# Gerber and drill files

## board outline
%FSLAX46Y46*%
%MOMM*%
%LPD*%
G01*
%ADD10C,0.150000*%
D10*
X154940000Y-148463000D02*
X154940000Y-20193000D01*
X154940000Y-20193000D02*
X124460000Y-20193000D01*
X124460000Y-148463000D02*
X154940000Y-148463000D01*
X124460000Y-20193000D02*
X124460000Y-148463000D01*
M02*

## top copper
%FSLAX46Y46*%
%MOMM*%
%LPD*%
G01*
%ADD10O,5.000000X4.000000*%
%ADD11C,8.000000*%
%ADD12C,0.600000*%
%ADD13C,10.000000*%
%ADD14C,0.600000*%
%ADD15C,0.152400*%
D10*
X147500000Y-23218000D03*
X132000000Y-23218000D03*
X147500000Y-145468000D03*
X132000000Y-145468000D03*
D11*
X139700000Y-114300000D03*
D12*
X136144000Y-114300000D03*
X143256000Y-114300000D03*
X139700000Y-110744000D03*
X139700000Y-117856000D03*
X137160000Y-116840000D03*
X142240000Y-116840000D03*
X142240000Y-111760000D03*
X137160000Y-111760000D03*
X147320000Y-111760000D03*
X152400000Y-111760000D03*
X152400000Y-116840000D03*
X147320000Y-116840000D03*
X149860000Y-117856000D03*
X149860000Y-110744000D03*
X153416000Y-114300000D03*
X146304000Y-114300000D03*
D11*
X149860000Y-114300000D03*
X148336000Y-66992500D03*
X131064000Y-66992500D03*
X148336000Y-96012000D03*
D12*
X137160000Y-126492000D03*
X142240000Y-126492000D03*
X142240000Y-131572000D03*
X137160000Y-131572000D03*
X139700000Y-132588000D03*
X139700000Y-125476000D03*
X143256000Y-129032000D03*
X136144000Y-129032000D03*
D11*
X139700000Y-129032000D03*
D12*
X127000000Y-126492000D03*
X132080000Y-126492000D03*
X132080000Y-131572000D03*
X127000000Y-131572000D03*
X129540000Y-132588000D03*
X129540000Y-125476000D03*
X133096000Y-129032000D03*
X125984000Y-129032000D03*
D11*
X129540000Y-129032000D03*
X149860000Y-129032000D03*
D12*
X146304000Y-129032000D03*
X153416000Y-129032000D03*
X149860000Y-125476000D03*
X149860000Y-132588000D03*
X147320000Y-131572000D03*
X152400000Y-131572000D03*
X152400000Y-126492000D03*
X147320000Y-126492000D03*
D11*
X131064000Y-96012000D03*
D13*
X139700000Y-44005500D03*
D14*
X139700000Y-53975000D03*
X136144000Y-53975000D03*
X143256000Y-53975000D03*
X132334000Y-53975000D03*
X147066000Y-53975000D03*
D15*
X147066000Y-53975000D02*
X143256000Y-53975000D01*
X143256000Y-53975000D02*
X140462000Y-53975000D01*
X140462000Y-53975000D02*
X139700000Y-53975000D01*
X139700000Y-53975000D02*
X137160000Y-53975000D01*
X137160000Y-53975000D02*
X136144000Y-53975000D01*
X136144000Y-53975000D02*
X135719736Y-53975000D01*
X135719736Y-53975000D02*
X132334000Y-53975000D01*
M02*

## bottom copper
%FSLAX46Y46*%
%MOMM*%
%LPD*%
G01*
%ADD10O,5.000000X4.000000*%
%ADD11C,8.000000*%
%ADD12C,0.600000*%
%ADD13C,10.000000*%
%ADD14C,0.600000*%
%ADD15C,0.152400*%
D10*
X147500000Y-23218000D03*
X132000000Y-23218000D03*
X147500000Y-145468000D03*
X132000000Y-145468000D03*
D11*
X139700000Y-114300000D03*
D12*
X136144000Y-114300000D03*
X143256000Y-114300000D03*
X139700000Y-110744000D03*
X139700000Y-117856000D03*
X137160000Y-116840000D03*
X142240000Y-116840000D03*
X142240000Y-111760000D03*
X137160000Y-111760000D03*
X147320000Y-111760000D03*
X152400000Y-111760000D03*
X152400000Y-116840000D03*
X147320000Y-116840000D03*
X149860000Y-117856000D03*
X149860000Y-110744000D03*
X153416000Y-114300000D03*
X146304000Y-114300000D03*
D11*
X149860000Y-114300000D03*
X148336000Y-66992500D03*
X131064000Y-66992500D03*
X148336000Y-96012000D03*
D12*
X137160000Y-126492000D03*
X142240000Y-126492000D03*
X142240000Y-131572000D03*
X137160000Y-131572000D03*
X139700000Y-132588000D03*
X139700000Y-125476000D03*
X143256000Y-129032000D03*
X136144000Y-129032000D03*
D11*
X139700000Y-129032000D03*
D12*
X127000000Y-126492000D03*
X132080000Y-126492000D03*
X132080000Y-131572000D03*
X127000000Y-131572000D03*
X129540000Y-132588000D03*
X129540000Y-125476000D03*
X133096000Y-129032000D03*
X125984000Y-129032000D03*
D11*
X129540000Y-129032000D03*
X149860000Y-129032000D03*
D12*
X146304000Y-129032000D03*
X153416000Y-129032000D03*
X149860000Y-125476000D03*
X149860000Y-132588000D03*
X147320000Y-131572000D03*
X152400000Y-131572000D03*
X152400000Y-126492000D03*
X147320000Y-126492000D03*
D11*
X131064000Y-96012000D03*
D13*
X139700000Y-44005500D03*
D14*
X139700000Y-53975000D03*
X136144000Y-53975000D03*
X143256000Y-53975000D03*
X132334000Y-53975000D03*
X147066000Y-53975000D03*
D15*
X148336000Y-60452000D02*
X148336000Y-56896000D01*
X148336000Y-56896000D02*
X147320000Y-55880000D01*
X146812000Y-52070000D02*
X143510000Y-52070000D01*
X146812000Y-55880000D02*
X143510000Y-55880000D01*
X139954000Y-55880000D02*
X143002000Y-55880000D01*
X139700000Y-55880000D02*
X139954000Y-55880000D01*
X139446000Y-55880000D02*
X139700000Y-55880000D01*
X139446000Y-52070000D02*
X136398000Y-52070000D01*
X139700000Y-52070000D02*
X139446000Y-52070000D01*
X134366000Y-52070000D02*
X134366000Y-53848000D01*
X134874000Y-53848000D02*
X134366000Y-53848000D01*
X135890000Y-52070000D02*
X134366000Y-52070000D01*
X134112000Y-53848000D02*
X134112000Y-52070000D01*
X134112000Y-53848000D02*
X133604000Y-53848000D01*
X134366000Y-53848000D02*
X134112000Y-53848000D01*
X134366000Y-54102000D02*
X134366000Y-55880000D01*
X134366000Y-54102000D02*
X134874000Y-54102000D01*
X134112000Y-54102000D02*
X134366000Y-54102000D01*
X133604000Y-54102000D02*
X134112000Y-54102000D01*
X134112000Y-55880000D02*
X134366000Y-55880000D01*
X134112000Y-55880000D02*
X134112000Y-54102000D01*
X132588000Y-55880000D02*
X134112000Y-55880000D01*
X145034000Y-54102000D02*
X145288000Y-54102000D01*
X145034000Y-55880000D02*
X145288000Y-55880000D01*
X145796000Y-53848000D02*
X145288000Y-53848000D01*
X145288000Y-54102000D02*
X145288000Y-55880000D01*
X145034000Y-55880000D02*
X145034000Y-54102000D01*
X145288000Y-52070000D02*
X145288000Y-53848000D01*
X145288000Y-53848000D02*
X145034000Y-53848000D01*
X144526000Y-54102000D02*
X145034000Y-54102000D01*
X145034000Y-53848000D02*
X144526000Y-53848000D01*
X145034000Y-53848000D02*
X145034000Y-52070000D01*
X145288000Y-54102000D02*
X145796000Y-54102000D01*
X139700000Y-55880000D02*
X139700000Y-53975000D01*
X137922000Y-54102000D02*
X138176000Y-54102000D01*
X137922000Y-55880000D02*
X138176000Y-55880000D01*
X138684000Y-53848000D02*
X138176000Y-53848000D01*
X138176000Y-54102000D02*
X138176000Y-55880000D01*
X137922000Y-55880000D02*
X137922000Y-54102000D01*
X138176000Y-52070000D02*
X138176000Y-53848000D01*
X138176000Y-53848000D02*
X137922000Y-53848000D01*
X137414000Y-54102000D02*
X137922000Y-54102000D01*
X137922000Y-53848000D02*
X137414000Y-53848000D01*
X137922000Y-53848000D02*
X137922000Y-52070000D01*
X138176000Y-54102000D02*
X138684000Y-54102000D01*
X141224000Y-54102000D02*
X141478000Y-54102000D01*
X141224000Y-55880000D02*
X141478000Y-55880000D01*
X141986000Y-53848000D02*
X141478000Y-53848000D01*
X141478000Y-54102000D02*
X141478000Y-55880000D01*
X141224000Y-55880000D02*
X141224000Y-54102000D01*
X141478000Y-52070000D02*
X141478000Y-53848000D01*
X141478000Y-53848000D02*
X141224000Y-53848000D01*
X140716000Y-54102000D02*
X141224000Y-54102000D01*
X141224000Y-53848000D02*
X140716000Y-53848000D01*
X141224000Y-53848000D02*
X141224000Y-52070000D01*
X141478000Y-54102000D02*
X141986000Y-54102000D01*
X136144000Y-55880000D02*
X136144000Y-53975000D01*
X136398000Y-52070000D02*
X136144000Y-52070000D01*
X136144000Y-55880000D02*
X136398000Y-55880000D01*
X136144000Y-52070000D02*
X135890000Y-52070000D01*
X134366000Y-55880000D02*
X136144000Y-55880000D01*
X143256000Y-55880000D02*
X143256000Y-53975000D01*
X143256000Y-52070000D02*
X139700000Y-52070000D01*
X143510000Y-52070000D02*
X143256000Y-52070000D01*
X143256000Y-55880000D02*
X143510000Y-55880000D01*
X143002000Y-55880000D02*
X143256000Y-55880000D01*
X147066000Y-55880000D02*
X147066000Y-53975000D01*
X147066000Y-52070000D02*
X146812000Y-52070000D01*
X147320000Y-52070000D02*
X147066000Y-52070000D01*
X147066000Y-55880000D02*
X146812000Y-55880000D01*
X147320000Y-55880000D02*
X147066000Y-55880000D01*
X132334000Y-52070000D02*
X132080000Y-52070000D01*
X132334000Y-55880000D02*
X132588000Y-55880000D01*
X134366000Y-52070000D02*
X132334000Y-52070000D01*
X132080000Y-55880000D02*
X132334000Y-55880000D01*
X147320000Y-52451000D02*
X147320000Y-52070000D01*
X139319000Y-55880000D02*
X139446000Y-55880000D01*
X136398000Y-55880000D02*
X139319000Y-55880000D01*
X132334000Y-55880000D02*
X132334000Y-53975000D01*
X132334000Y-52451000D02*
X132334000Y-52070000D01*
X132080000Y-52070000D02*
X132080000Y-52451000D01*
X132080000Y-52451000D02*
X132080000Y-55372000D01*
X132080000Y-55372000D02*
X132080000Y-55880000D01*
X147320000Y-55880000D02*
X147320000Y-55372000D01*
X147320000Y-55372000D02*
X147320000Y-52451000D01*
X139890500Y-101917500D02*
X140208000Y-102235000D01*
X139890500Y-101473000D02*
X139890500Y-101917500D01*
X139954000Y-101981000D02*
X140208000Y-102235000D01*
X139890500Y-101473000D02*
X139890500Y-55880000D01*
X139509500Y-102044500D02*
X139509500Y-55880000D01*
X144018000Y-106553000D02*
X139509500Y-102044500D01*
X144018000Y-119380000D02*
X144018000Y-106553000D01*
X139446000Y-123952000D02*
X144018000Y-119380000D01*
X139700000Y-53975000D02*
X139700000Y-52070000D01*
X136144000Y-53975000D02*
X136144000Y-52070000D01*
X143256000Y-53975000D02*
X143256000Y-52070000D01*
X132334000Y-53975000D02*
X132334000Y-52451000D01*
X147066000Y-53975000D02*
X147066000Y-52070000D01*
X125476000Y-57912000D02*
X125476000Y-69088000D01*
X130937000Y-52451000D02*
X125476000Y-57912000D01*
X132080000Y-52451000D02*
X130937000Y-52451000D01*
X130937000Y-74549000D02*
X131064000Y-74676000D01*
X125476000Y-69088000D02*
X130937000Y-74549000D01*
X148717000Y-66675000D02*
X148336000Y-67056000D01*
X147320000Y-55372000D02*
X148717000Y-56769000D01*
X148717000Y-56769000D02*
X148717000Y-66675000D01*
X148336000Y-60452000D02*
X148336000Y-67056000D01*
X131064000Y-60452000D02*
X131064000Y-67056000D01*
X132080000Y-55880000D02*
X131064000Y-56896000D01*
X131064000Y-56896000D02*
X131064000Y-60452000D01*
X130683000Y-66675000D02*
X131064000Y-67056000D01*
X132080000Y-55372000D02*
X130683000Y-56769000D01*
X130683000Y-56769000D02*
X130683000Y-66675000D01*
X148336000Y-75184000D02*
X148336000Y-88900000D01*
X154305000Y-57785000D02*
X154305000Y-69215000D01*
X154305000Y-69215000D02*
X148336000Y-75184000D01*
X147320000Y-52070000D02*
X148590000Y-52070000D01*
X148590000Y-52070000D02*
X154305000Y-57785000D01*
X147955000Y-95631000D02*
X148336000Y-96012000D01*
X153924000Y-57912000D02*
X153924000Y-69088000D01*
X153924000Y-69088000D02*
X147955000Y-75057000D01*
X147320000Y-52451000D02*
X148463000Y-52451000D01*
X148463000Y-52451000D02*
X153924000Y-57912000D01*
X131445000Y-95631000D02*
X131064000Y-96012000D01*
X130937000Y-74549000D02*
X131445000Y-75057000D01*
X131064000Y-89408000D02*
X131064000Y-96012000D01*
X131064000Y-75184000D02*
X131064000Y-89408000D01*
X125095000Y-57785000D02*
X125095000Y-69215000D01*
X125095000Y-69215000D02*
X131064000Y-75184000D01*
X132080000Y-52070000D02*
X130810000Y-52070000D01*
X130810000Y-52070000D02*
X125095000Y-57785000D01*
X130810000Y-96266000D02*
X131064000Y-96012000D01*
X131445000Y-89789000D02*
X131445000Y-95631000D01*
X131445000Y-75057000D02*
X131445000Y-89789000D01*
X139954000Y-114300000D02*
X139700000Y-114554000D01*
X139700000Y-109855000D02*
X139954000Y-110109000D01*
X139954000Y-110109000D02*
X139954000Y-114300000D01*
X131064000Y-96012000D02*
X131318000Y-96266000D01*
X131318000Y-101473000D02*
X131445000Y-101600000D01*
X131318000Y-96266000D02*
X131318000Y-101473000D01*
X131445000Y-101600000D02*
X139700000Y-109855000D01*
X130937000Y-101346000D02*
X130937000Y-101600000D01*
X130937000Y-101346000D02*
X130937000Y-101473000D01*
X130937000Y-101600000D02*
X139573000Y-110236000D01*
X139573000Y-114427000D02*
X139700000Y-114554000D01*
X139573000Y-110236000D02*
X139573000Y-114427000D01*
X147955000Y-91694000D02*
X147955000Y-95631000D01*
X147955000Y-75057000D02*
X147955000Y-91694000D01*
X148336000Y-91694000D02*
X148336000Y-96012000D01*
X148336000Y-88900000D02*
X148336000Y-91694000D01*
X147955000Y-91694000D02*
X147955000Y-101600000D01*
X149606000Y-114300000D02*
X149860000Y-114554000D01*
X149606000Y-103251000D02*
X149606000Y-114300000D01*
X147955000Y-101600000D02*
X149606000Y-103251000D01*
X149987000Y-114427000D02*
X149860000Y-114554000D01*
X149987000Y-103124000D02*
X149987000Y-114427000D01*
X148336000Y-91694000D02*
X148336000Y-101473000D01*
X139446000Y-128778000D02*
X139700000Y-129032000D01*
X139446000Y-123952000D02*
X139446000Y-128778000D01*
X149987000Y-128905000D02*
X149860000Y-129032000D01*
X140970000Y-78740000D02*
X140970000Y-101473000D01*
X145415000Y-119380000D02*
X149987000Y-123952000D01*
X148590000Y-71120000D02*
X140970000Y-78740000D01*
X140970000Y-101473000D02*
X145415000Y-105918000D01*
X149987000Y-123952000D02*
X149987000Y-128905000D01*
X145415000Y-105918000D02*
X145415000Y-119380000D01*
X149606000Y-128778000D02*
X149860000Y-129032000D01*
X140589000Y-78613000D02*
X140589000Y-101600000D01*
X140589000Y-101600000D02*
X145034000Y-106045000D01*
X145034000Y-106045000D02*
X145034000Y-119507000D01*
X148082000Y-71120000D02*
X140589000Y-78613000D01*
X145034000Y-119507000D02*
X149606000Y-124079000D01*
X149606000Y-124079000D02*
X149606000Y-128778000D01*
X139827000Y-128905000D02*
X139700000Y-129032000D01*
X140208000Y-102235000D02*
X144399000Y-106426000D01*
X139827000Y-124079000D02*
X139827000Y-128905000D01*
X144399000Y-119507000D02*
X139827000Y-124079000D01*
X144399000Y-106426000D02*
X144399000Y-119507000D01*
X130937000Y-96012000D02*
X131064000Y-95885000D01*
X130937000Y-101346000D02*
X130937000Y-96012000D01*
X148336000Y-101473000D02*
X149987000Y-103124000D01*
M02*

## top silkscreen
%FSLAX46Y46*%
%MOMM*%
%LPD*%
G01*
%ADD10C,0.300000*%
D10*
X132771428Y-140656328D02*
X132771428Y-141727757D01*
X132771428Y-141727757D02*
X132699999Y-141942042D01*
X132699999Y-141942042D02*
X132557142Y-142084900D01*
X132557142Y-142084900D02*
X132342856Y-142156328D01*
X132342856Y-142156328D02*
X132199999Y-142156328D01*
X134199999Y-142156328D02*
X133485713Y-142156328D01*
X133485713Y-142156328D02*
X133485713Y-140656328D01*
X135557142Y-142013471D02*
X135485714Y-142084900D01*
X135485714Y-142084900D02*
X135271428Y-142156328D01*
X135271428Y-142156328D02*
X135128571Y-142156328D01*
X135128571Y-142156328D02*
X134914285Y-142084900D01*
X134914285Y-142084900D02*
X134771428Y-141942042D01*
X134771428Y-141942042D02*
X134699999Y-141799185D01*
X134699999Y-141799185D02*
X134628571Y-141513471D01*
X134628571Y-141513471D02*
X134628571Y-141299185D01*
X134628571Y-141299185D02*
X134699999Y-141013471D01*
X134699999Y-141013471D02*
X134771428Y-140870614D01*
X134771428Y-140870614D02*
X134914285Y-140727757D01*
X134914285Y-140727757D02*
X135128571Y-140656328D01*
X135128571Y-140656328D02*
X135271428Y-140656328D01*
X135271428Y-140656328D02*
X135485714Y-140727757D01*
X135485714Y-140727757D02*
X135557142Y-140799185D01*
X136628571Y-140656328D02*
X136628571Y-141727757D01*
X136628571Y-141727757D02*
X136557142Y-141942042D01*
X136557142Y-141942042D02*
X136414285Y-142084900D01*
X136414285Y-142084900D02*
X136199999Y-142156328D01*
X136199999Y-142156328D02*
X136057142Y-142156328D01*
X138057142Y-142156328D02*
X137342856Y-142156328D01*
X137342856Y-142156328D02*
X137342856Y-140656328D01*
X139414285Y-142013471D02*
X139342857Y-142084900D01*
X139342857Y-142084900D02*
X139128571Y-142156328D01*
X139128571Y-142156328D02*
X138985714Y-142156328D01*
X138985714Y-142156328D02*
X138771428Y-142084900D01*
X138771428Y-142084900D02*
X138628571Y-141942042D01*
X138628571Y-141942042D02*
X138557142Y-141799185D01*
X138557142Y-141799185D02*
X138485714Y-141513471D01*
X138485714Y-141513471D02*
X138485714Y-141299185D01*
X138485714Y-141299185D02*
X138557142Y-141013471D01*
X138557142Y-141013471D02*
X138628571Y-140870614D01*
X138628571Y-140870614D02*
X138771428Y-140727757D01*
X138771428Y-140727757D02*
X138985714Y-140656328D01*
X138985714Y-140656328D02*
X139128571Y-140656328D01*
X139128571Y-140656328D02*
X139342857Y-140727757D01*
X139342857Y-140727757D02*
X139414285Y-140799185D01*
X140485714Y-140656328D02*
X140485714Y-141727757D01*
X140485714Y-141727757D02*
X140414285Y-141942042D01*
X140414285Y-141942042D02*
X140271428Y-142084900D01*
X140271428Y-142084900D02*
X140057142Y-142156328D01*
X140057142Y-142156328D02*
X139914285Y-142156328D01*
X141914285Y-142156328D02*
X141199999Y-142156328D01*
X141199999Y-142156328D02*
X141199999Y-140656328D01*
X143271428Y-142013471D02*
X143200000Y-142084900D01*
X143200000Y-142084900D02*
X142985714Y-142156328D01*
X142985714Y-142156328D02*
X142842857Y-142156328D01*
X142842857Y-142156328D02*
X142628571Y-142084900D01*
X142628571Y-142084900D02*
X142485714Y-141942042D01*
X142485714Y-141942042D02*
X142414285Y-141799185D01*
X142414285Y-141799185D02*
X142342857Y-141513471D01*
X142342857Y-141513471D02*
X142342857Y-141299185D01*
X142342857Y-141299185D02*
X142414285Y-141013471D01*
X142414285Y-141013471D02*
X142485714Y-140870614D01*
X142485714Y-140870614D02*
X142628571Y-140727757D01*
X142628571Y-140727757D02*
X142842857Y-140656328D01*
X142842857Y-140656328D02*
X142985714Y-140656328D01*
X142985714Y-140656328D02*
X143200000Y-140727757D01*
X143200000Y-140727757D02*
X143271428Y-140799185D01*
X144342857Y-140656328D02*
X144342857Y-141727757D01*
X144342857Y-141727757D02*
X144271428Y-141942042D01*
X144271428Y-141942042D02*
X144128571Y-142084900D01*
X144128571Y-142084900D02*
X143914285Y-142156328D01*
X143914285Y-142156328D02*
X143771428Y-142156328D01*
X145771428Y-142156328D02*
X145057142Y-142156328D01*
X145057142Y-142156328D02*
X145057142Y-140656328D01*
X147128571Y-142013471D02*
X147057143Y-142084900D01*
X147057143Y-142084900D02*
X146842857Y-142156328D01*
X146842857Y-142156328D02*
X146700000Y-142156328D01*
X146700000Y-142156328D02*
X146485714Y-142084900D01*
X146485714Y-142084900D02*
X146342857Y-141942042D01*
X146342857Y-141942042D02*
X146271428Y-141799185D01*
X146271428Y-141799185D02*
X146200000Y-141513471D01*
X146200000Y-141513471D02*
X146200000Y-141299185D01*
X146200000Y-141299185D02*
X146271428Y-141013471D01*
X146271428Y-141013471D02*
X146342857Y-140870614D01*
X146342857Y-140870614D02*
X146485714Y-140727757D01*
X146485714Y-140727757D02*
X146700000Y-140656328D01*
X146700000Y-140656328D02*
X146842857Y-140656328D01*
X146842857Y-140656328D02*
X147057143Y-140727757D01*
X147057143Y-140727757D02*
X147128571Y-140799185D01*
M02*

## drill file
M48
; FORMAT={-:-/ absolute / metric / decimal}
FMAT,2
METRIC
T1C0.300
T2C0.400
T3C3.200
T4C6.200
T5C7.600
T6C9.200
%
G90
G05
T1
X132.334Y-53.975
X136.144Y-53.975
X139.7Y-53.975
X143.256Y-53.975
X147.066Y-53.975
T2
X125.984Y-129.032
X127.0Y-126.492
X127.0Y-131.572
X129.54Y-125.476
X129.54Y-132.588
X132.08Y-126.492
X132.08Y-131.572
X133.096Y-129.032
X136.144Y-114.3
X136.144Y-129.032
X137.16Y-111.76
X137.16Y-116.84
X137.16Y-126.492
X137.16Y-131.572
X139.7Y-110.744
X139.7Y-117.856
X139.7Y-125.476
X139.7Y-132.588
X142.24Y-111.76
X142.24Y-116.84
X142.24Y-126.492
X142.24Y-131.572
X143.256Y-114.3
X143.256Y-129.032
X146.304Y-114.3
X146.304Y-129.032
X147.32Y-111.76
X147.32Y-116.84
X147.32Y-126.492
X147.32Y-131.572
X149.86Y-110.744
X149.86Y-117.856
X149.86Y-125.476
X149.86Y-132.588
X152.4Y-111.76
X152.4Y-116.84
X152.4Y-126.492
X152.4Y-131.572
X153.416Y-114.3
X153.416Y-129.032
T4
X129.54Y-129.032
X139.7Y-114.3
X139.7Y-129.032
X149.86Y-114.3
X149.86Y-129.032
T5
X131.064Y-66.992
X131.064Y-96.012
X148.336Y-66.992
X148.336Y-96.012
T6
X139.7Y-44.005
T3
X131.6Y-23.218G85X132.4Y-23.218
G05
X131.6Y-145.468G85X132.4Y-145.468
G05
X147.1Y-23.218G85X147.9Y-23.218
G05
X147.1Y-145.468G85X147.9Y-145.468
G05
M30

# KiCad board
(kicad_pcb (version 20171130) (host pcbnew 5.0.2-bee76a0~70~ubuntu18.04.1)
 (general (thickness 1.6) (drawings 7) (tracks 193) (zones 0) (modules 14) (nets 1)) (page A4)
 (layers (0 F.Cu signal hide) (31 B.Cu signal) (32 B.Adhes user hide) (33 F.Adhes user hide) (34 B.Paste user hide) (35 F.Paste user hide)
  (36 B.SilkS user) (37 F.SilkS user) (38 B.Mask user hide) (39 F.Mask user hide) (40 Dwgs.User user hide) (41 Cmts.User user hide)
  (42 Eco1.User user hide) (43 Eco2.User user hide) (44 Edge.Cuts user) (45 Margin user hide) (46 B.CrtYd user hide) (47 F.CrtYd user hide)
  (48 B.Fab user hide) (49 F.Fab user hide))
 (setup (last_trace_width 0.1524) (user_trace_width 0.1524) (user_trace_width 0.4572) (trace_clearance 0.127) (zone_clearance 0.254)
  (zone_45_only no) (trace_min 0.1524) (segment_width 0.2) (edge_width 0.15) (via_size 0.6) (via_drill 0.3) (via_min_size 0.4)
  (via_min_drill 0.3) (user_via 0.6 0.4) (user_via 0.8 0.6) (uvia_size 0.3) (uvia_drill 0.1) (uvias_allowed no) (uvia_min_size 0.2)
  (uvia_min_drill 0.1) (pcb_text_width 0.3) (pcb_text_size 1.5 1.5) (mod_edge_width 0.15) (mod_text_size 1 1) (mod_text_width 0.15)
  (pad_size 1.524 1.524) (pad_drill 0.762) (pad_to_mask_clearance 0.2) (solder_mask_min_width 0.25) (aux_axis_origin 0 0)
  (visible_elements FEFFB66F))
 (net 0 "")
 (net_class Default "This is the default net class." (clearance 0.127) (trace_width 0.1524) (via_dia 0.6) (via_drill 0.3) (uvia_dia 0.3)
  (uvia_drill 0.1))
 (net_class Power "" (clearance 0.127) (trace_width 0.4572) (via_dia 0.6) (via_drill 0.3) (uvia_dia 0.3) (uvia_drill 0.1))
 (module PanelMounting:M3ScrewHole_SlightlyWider (layer F.Cu) (at 147.5 23.218)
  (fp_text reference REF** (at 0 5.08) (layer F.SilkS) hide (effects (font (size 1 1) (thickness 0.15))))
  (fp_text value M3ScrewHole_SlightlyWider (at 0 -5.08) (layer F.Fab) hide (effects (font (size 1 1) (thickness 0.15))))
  (pad 1 thru_hole oval (at 0 0) (size 5 4) (drill oval 4 3.2) (layers *.Cu *.Mask)))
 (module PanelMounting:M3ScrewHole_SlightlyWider (layer F.Cu) (at 132 23.218)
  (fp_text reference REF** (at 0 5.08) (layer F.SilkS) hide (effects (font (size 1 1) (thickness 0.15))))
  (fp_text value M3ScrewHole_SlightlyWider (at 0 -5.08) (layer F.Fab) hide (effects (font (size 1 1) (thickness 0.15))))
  (pad 1 thru_hole oval (at 0 0) (size 5 4) (drill oval 4 3.2) (layers *.Cu *.Mask)))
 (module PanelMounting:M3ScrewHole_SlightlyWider (layer F.Cu) (at 147.5 145.468)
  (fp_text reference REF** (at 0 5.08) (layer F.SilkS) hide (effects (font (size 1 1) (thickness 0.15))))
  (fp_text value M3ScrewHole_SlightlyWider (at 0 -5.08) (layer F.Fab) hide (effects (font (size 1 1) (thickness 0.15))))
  (pad 1 thru_hole oval (at 0 0) (size 5 4) (drill oval 4 3.2) (layers *.Cu *.Mask)))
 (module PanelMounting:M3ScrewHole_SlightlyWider (layer F.Cu) (at 132 145.468)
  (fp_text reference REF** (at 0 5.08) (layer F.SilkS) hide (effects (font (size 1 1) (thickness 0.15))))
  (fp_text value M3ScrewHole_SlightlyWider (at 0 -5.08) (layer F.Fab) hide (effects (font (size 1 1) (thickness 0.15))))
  (pad 1 thru_hole oval (at 0 0) (size 5 4) (drill oval 4 3.2) (layers *.Cu *.Mask)))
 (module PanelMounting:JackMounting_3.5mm (layer B.Cu) (at 139.7 114.3 180)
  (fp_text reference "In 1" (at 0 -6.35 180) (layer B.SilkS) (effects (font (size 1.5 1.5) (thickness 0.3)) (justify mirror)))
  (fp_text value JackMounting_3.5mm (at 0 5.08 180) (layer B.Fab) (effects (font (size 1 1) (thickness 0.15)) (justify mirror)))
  (pad 1 thru_hole circle (at 0 0 180) (size 8 8) (drill 6.2) (layers *.Cu *.Mask))
  (pad "" thru_hole circle (at 3.556 0 180) (size 0.6 0.6) (drill 0.4) (layers *.Cu *.Mask))
  (pad "" thru_hole circle (at -3.556 0 180) (size 0.6 0.6) (drill 0.4) (layers *.Cu *.Mask))
  (pad "" thru_hole circle (at 0 3.556 180) (size 0.6 0.6) (drill 0.4) (layers *.Cu *.Mask))
  (pad "" thru_hole circle (at 0 -3.556 180) (size 0.6 0.6) (drill 0.4) (layers *.Cu *.Mask))
  (pad "" thru_hole circle (at 2.54 -2.54 180) (size 0.6 0.6) (drill 0.4) (layers *.Cu *.Mask))
  (pad "" thru_hole circle (at -2.54 -2.54 180) (size 0.6 0.6) (drill 0.4) (layers *.Cu *.Mask))
  (pad "" thru_hole circle (at -2.54 2.54 180) (size 0.6 0.6) (drill 0.4) (layers *.Cu *.Mask))
  (pad "" thru_hole circle (at 2.54 2.54 180) (size 0.6 0.6) (drill 0.4) (layers *.Cu *.Mask)))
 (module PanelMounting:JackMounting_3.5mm (layer B.Cu) (at 149.86 114.3 180)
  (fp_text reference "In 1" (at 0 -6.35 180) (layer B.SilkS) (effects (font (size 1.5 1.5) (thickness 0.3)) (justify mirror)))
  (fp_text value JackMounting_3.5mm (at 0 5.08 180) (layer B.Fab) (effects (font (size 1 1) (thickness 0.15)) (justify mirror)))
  (pad "" thru_hole circle (at 2.54 2.54 180) (size 0.6 0.6) (drill 0.4) (layers *.Cu *.Mask))
  (pad "" thru_hole circle (at -2.54 2.54 180) (size 0.6 0.6) (drill 0.4) (layers *.Cu *.Mask))
  (pad "" thru_hole circle (at -2.54 -2.54 180) (size 0.6 0.6) (drill 0.4) (layers *.Cu *.Mask))
  (pad "" thru_hole circle (at 2.54 -2.54 180) (size 0.6 0.6) (drill 0.4) (layers *.Cu *.Mask))
  (pad "" thru_hole circle (at 0 -3.556 180) (size 0.6 0.6) (drill 0.4) (layers *.Cu *.Mask))
  (pad "" thru_hole circle (at 0 3.556 180) (size 0.6 0.6) (drill 0.4) (layers *.Cu *.Mask))
  (pad "" thru_hole circle (at -3.556 0 180) (size 0.6 0.6) (drill 0.4) (layers *.Cu *.Mask))
  (pad "" thru_hole circle (at 3.556 0 180) (size 0.6 0.6) (drill 0.4) (layers *.Cu *.Mask))
  (pad 1 thru_hole circle (at 0 0 180) (size 8 8) (drill 6.2) (layers *.Cu *.Mask)))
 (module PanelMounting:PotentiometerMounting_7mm (layer B.Cu) (at 148.336 66.9925 180)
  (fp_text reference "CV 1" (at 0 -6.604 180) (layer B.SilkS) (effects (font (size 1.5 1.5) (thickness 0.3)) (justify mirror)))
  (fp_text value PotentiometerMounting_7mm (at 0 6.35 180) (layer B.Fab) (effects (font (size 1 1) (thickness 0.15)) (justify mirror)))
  (pad 1 thru_hole circle (at 0 0 180) (size 8 8) (drill 7.6) (layers *.Cu *.Mask)))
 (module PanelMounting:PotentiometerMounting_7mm (layer B.Cu) (at 131.064 66.9925 180)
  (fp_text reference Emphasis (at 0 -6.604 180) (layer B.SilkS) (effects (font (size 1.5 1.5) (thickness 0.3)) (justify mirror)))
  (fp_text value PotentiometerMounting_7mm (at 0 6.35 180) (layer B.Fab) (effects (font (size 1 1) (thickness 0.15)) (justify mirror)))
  (pad 1 thru_hole circle (at 0 0 180) (size 8 8) (drill 7.6) (layers *.Cu *.Mask)))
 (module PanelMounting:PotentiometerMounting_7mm (layer B.Cu) (at 148.336 96.012 180)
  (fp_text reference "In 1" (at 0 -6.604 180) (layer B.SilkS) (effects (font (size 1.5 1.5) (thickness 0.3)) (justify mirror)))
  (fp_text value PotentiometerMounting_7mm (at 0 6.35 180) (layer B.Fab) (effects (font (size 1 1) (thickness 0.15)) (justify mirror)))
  (pad 1 thru_hole circle (at 0 0 180) (size 8 8) (drill 7.6) (layers *.Cu *.Mask)))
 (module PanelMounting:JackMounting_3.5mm (layer B.Cu) (at 139.7 129.032 180)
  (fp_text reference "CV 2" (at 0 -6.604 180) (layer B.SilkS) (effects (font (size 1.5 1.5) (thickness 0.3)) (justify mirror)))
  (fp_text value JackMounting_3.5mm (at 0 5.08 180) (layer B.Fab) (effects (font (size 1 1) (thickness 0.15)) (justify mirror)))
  (pad "" thru_hole circle (at 2.54 2.54 180) (size 0.6 0.6) (drill 0.4) (layers *.Cu *.Mask))
  (pad "" thru_hole circle (at -2.54 2.54 180) (size 0.6 0.6) (drill 0.4) (layers *.Cu *.Mask))
  (pad "" thru_hole circle (at -2.54 -2.54 180) (size 0.6 0.6) (drill 0.4) (layers *.Cu *.Mask))
  (pad "" thru_hole circle (at 2.54 -2.54 180) (size 0.6 0.6) (drill 0.4) (layers *.Cu *.Mask))
  (pad "" thru_hole circle (at 0 -3.556 180) (size 0.6 0.6) (drill 0.4) (layers *.Cu *.Mask))
  (pad "" thru_hole circle (at 0 3.556 180) (size 0.6 0.6) (drill 0.4) (layers *.Cu *.Mask))
  (pad "" thru_hole circle (at -3.556 0 180) (size 0.6 0.6) (drill 0.4) (layers *.Cu *.Mask))
  (pad "" thru_hole circle (at 3.556 0 180) (size 0.6 0.6) (drill 0.4) (layers *.Cu *.Mask))
  (pad 1 thru_hole circle (at 0 0 180) (size 8 8) (drill 6.2) (layers *.Cu *.Mask)))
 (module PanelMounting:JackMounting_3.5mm (layer B.Cu) (at 129.54 129.032 180)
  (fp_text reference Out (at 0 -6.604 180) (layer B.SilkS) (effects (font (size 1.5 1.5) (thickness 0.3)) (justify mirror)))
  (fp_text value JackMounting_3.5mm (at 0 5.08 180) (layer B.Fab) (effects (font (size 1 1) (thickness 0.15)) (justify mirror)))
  (pad "" thru_hole circle (at 2.54 2.54 180) (size 0.6 0.6) (drill 0.4) (layers *.Cu *.Mask))
  (pad "" thru_hole circle (at -2.54 2.54 180) (size 0.6 0.6) (drill 0.4) (layers *.Cu *.Mask))
  (pad "" thru_hole circle (at -2.54 -2.54 180) (size 0.6 0.6) (drill 0.4) (layers *.Cu *.Mask))
  (pad "" thru_hole circle (at 2.54 -2.54 180) (size 0.6 0.6) (drill 0.4) (layers *.Cu *.Mask))
  (pad "" thru_hole circle (at 0 -3.556 180) (size 0.6 0.6) (drill 0.4) (layers *.Cu *.Mask))
  (pad "" thru_hole circle (at 0 3.556 180) (size 0.6 0.6) (drill 0.4) (layers *.Cu *.Mask))
  (pad "" thru_hole circle (at -3.556 0 180) (size 0.6 0.6) (drill 0.4) (layers *.Cu *.Mask))
  (pad "" thru_hole circle (at 3.556 0 180) (size 0.6 0.6) (drill 0.4) (layers *.Cu *.Mask))
  (pad 1 thru_hole circle (at 0 0 180) (size 8 8) (drill 6.2) (layers *.Cu *.Mask)))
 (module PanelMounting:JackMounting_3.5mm (layer B.Cu) (at 149.86 129.032 180)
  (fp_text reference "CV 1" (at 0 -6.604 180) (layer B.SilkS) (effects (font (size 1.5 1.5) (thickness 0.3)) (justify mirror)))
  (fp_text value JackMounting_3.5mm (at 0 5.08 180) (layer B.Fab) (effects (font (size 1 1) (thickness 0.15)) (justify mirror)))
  (pad 1 thru_hole circle (at 0 0 180) (size 8 8) (drill 6.2) (layers *.Cu *.Mask))
  (pad "" thru_hole circle (at 3.556 0 180) (size 0.6 0.6) (drill 0.4) (layers *.Cu *.Mask))
  (pad "" thru_hole circle (at -3.556 0 180) (size 0.6 0.6) (drill 0.4) (layers *.Cu *.Mask))
  (pad "" thru_hole circle (at 0 3.556 180) (size 0.6 0.6) (drill 0.4) (layers *.Cu *.Mask))
  (pad "" thru_hole circle (at 0 -3.556 180) (size 0.6 0.6) (drill 0.4) (layers *.Cu *.Mask))
  (pad "" thru_hole circle (at 2.54 -2.54 180) (size 0.6 0.6) (drill 0.4) (layers *.Cu *.Mask))
  (pad "" thru_hole circle (at -2.54 -2.54 180) (size 0.6 0.6) (drill 0.4) (layers *.Cu *.Mask))
  (pad "" thru_hole circle (at -2.54 2.54 180) (size 0.6 0.6) (drill 0.4) (layers *.Cu *.Mask))
  (pad "" thru_hole circle (at 2.54 2.54 180) (size 0.6 0.6) (drill 0.4) (layers *.Cu *.Mask)))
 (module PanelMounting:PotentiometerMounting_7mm (layer B.Cu) (at 131.064 96.012 180)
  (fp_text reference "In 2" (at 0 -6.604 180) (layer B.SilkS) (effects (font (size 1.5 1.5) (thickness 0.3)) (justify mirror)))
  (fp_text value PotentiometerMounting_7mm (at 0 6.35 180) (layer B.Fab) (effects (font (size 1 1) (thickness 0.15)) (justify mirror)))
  (pad 1 thru_hole circle (at 0 0 180) (size 8 8) (drill 7.6) (layers *.Cu *.Mask)))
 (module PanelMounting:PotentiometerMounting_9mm (layer B.Cu) (at 139.7 44.0055 180)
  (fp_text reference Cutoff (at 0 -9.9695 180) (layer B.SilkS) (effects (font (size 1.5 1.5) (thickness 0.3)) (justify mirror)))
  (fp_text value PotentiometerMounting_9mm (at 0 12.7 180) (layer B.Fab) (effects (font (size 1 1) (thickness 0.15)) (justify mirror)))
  (pad 1 thru_hole circle (at 0 0 180) (size 10 10) (drill 9.2) (layers *.Cu *.Mask)))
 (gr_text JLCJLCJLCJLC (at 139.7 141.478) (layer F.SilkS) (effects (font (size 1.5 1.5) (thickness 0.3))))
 (gr_line (start 154.94 148.463) (end 154.94 20.193) (layer Edge.Cuts) (width 0.15))
 (gr_line (start 154.94 20.193) (end 124.46 20.193) (layer Edge.Cuts) (width 0.15))
 (gr_line (start 124.46 148.463) (end 154.94 148.463) (layer Edge.Cuts) (width 0.15))
 (gr_line (start 124.46 20.193) (end 124.46 148.463) (layer Edge.Cuts) (width 0.15))
 (segment (start 148.336 60.452) (end 148.336 56.896) (width 0.1524) (layer B.Cu) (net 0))
 (segment (start 148.336 56.896) (end 147.32 55.88) (width 0.1524) (layer B.Cu) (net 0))
 (segment (start 146.812 52.07) (end 143.51 52.07) (width 0.1524) (layer B.Cu) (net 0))
 (segment (start 146.812 55.88) (end 143.51 55.88) (width 0.1524) (layer B.Cu) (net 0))
 (segment (start 139.954 55.88) (end 143.002 55.88) (width 0.1524) (layer B.Cu) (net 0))
 (segment (start 139.7 55.88) (end 139.954 55.88) (width 0.1524) (layer B.Cu) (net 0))
 (segment (start 139.446 55.88) (end 139.7 55.88) (width 0.1524) (layer B.Cu) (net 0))
 (segment (start 139.446 52.07) (end 136.398 52.07) (width 0.1524) (layer B.Cu) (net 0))
 (segment (start 139.7 52.07) (end 139.446 52.07) (width 0.1524) (layer B.Cu) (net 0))
 (segment (start 134.366 52.07) (end 134.366 53.848) (width 0.1524) (layer B.Cu) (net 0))
 (segment (start 134.874 53.848) (end 134.366 53.848) (width 0.1524) (layer B.Cu) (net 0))
 (segment (start 135.89 52.07) (end 134.366 52.07) (width 0.1524) (layer B.Cu) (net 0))
 (segment (start 134.112 53.848) (end 134.112 52.07) (width 0.1524) (layer B.Cu) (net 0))
 (segment (start 134.112 53.848) (end 133.604 53.848) (width 0.1524) (layer B.Cu) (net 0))
 (segment (start 134.366 53.848) (end 134.112 53.848) (width 0.1524) (layer B.Cu) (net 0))
 (segment (start 134.366 54.102) (end 134.366 55.88) (width 0.1524) (layer B.Cu) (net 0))
 (segment (start 134.366 54.102) (end 134.874 54.102) (width 0.1524) (layer B.Cu) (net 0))
 (segment (start 134.112 54.102) (end 134.366 54.102) (width 0.1524) (layer B.Cu) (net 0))
 (segment (start 133.604 54.102) (end 134.112 54.102) (width 0.1524) (layer B.Cu) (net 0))
 (segment (start 134.112 55.88) (end 134.366 55.88) (width 0.1524) (layer B.Cu) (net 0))
 (segment (start 134.112 55.88) (end 134.112 54.102) (width 0.1524) (layer B.Cu) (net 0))
 (segment (start 132.588 55.88) (end 134.112 55.88) (width 0.1524) (layer B.Cu) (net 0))
 (segment (start 145.034 54.102) (end 145.288 54.102) (width 0.1524) (layer B.Cu) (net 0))
 (segment (start 145.034 55.88) (end 145.288 55.88) (width 0.1524) (layer B.Cu) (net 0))
 (segment (start 145.796 53.848) (end 145.288 53.848) (width 0.1524) (layer B.Cu) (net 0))
 (segment (start 145.288 54.102) (end 145.288 55.88) (width 0.1524) (layer B.Cu) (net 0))
 (segment (start 145.034 55.88) (end 145.034 54.102) (width 0.1524) (layer B.Cu) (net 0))
 (segment (start 145.288 52.07) (end 145.288 53.848) (width 0.1524) (layer B.Cu) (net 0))
 (segment (start 145.288 53.848) (end 145.034 53.848) (width 0.1524) (layer B.Cu) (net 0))
 (segment (start 144.526 54.102) (end 145.034 54.102) (width 0.1524) (layer B.Cu) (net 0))
 (segment (start 145.034 53.848) (end 144.526 53.848) (width 0.1524) (layer B.Cu) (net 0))
 (segment (start 145.034 53.848) (end 145.034 52.07) (width 0.1524) (layer B.Cu) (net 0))
 (segment (start 145.288 54.102) (end 145.796 54.102) (width 0.1524) (layer B.Cu) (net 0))
 (segment (start 139.7 55.88) (end 139.7 53.975) (width 0.1524) (layer B.Cu) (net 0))
 (segment (start 137.922 54.102) (end 138.176 54.102) (width 0.1524) (layer B.Cu) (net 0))
 (segment (start 137.922 55.88) (end 138.176 55.88) (width 0.1524) (layer B.Cu) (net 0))
 (segment (start 138.684 53.848) (end 138.176 53.848) (width 0.1524) (layer B.Cu) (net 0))
 (segment (start 138.176 54.102) (end 138.176 55.88) (width 0.1524) (layer B.Cu) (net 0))
 (segment (start 137.922 55.88) (end 137.922 54.102) (width 0.1524) (layer B.Cu) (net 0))
 (segment (start 138.176 52.07) (end 138.176 53.848) (width 0.1524) (layer B.Cu) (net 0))
 (segment (start 138.176 53.848) (end 137.922 53.848) (width 0.1524) (layer B.Cu) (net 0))
 (segment (start 137.414 54.102) (end 137.922 54.102) (width 0.1524) (layer B.Cu) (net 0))
 (segment (start 137.922 53.848) (end 137.414 53.848) (width 0.1524) (layer B.Cu) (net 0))
 (segment (start 137.922 53.848) (end 137.922 52.07) (width 0.1524) (layer B.Cu) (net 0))
 (segment (start 138.176 54.102) (end 138.684 54.102) (width 0.1524) (layer B.Cu) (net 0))
 (segment (start 141.224 54.102) (end 141.478 54.102) (width 0.1524) (layer B.Cu) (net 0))
 (segment (start 141.224 55.88) (end 141.478 55.88) (width 0.1524) (layer B.Cu) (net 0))
 (segment (start 141.986 53.848) (end 141.478 53.848) (width 0.1524) (layer B.Cu) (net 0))
 (segment (start 141.478 54.102) (end 141.478 55.88) (width 0.1524) (layer B.Cu) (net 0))
 (segment (start 141.224 55.88) (end 141.224 54.102) (width 0.1524) (layer B.Cu) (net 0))
 (segment (start 141.478 52.07) (end 141.478 53.848) (width 0.1524) (layer B.Cu) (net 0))
 (segment (start 141.478 53.848) (end 141.224 53.848) (width 0.1524) (layer B.Cu) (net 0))
 (segment (start 140.716 54.102) (end 141.224 54.102) (width 0.1524) (layer B.Cu) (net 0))
 (segment (start 141.224 53.848) (end 140.716 53.848) (width 0.1524) (layer B.Cu) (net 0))
 (segment (start 141.224 53.848) (end 141.224 52.07) (width 0.1524) (layer B.Cu) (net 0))
 (segment (start 141.478 54.102) (end 141.986 54.102) (width 0.1524) (layer B.Cu) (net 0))
 (segment (start 136.144 55.88) (end 136.144 53.975) (width 0.1524) (layer B.Cu) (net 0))
 (segment (start 136.398 52.07) (end 136.144 52.07) (width 0.1524) (layer B.Cu) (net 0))
 (segment (start 136.144 55.88) (end 136.398 55.88) (width 0.1524) (layer B.Cu) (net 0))
 (segment (start 136.144 52.07) (end 135.89 52.07) (width 0.1524) (layer B.Cu) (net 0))
 (segment (start 134.366 55.88) (end 136.144 55.88) (width 0.1524) (layer B.Cu) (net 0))
 (segment (start 143.256 55.88) (end 143.256 53.975) (width 0.1524) (layer B.Cu) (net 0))
 (segment (start 143.256 52.07) (end 139.7 52.07) (width 0.1524) (layer B.Cu) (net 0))
 (segment (start 143.51 52.07) (end 143.256 52.07) (width 0.1524) (layer B.Cu) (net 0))
 (segment (start 143.256 55.88) (end 143.51 55.88) (width 0.1524) (layer B.Cu) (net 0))
 (segment (start 143.002 55.88) (end 143.256 55.88) (width 0.1524) (layer B.Cu) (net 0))
 (segment (start 147.066 55.88) (end 147.066 53.975) (width 0.1524) (layer B.Cu) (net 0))
 (segment (start 147.066 52.07) (end 146.812 52.07) (width 0.1524) (layer B.Cu) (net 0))
 (segment (start 147.32 52.07) (end 147.066 52.07) (width 0.1524) (layer B.Cu) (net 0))
 (segment (start 147.066 55.88) (end 146.812 55.88) (width 0.1524) (layer B.Cu) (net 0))
 (segment (start 147.32 55.88) (end 147.066 55.88) (width 0.1524) (layer B.Cu) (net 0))
 (segment (start 132.334 52.07) (end 132.08 52.07) (width 0.1524) (layer B.Cu) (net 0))
 (segment (start 132.334 55.88) (end 132.588 55.88) (width 0.1524) (layer B.Cu) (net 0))
 (segment (start 134.366 52.07) (end 132.334 52.07) (width 0.1524) (layer B.Cu) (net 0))
 (segment (start 132.08 55.88) (end 132.334 55.88) (width 0.1524) (layer B.Cu) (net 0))
 (segment (start 147.32 52.451) (end 147.32 52.07) (width 0.1524) (layer B.Cu) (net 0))
 (segment (start 139.319 55.88) (end 139.446 55.88) (width 0.1524) (layer B.Cu) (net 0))
 (segment (start 136.398 55.88) (end 139.319 55.88) (width 0.1524) (layer B.Cu) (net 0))
 (segment (start 132.334 55.88) (end 132.334 53.975) (width 0.1524) (layer B.Cu) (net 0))
 (segment (start 132.334 52.451) (end 132.334 52.07) (width 0.1524) (layer B.Cu) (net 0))
 (segment (start 132.08 52.07) (end 132.08 52.451) (width 0.1524) (layer B.Cu) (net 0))
 (segment (start 132.08 52.451) (end 132.08 55.372) (width 0.1524) (layer B.Cu) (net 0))
 (segment (start 132.08 55.372) (end 132.08 55.88) (width 0.1524) (layer B.Cu) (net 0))
 (segment (start 147.32 55.88) (end 147.32 55.372) (width 0.1524) (layer B.Cu) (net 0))
 (segment (start 147.32 55.372) (end 147.32 52.451) (width 0.1524) (layer B.Cu) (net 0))
 (segment (start 139.8905 101.9175) (end 140.208 102.235) (width 0.1524) (layer B.Cu) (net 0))
 (segment (start 139.8905 101.473) (end 139.8905 101.9175) (width 0.1524) (layer B.Cu) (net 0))
 (segment (start 139.954 101.981) (end 140.208 102.235) (width 0.1524) (layer B.Cu) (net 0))
 (segment (start 139.8905 101.473) (end 139.8905 55.88) (width 0.1524) (layer B.Cu) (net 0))
 (segment (start 139.5095 102.0445) (end 139.5095 55.88) (width 0.1524) (layer B.Cu) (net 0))
 (segment (start 144.018 106.553) (end 139.5095 102.0445) (width 0.1524) (layer B.Cu) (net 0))
 (segment (start 144.018 119.38) (end 144.018 106.553) (width 0.1524) (layer B.Cu) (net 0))
 (segment (start 139.446 123.952) (end 144.018 119.38) (width 0.1524) (layer B.Cu) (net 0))
 (segment (start 139.7 53.975) (end 139.7 52.07) (width 0.1524) (layer B.Cu) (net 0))
 (via (at 139.7 53.975) (size 0.6) (drill 0.3) (layers F.Cu B.Cu) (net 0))
 (segment (start 136.144 53.975) (end 136.144 52.07) (width 0.1524) (layer B.Cu) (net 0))
 (via (at 136.144 53.975) (size 0.6) (drill 0.3) (layers F.Cu B.Cu) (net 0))
 (segment (start 143.256 53.975) (end 143.256 52.07) (width 0.1524) (layer B.Cu) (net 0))
 (via (at 143.256 53.975) (size 0.6) (drill 0.3) (layers F.Cu B.Cu) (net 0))
 (segment (start 132.334 53.975) (end 132.334 52.451) (width 0.1524) (layer B.Cu) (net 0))
 (via (at 132.334 53.975) (size 0.6) (drill 0.3) (layers F.Cu B.Cu) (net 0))
 (segment (start 147.066 53.975) (end 147.066 52.07) (width 0.1524) (layer B.Cu) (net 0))
 (via (at 147.066 53.975) (size 0.6) (drill 0.3) (layers F.Cu B.Cu) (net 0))
 (segment (start 147.066 53.975) (end 143.256 53.975) (width 0.1524) (layer F.Cu) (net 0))
 (segment (start 143.256 53.975) (end 140.462 53.975) (width 0.1524) (layer F.Cu) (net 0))
 (segment (start 140.462 53.975) (end 139.7 53.975) (width 0.1524) (layer F.Cu) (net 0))
 (segment (start 139.7 53.975) (end 137.16 53.975) (width 0.1524) (layer F.Cu) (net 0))
 (segment (start 137.16 53.975) (end 136.144 53.975) (width 0.1524) (layer F.Cu) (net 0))
 (segment (start 136.144 53.975) (end 135.719736 53.975) (width 0.1524) (layer F.Cu) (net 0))
 (segment (start 135.719736 53.975) (end 132.334 53.975) (width 0.1524) (layer F.Cu) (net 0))
 (segment (start 125.476 57.912) (end 125.476 69.088) (width 0.1524) (layer B.Cu) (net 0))
 (segment (start 130.937 52.451) (end 125.476 57.912) (width 0.1524) (layer B.Cu) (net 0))
 (segment (start 132.08 52.451) (end 130.937 52.451) (width 0.1524) (layer B.Cu) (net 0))
 (segment (start 130.937 74.549) (end 131.064 74.676) (width 0.1524) (layer B.Cu) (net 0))
 (segment (start 125.476 69.088) (end 130.937 74.549) (width 0.1524) (layer B.Cu) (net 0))
 (segment (start 148.717 66.675) (end 148.336 67.056) (width 0.1524) (layer B.Cu) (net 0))
 (segment (start 147.32 55.372) (end 148.717 56.769) (width 0.1524) (layer B.Cu) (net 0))
 (segment (start 148.717 56.769) (end 148.717 66.675) (width 0.1524) (layer B.Cu) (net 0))
 (segment (start 148.336 60.452) (end 148.336 67.056) (width 0.1524) (layer B.Cu) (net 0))
 (segment (start 131.064 60.452) (end 131.064 67.056) (width 0.1524) (layer B.Cu) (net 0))
 (segment (start 132.08 55.88) (end 131.064 56.896) (width 0.1524) (layer B.Cu) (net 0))
 (segment (start 131.064 56.896) (end 131.064 60.452) (width 0.1524) (layer B.Cu) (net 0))
 (segment (start 130.683 66.675) (end 131.064 67.056) (width 0.1524) (layer B.Cu) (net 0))
 (segment (start 132.08 55.372) (end 130.683 56.769) (width 0.1524) (layer B.Cu) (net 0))
 (segment (start 130.683 56.769) (end 130.683 66.675) (width 0.1524) (layer B.Cu) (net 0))
 (segment (start 148.336 75.184) (end 148.336 88.9) (width 0.1524) (layer B.Cu) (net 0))
 (segment (start 154.305 57.785) (end 154.305 69.215) (width 0.1524) (layer B.Cu) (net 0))
 (segment (start 154.305 69.215) (end 148.336 75.184) (width 0.1524) (layer B.Cu) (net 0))
 (segment (start 147.32 52.07) (end 148.59 52.07) (width 0.1524) (layer B.Cu) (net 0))
 (segment (start 148.59 52.07) (end 154.305 57.785) (width 0.1524) (layer B.Cu) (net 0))
 (segment (start 147.955 95.631) (end 148.336 96.012) (width 0.1524) (layer B.Cu) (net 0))
 (segment (start 153.924 57.912) (end 153.924 69.088) (width 0.1524) (layer B.Cu) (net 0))
 (segment (start 153.924 69.088) (end 147.955 75.057) (width 0.1524) (layer B.Cu) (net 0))
 (segment (start 147.32 52.451) (end 148.463 52.451) (width 0.1524) (layer B.Cu) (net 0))
 (segment (start 148.463 52.451) (end 153.924 57.912) (width 0.1524) (layer B.Cu) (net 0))
 (segment (start 131.445 95.631) (end 131.064 96.012) (width 0.1524) (layer B.Cu) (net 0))
 (segment (start 130.937 74.549) (end 131.445 75.057) (width 0.1524) (layer B.Cu) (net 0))
 (segment (start 131.064 89.408) (end 131.064 96.012) (width 0.1524) (layer B.Cu) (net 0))
 (segment (start 131.064 75.184) (end 131.064 89.408) (width 0.1524) (layer B.Cu) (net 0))
 (segment (start 125.095 57.785) (end 125.095 69.215) (width 0.1524) (layer B.Cu) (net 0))
 (segment (start 125.095 69.215) (end 131.064 75.184) (width 0.1524) (layer B.Cu) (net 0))
 (segment (start 132.08 52.07) (end 130.81 52.07) (width 0.1524) (layer B.Cu) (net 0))
 (segment (start 130.81 52.07) (end 125.095 57.785) (width 0.1524) (layer B.Cu) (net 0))
 (segment (start 130.81 96.266) (end 131.064 96.012) (width 0.1524) (layer B.Cu) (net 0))
 (segment (start 131.445 89.789) (end 131.445 95.631) (width 0.1524) (layer B.Cu) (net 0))
 (segment (start 131.445 75.057) (end 131.445 89.789) (width 0.1524) (layer B.Cu) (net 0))
 (segment (start 139.954 114.3) (end 139.7 114.554) (width 0.1524) (layer B.Cu) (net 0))
 (segment (start 139.7 109.855) (end 139.954 110.109) (width 0.1524) (layer B.Cu) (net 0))
 (segment (start 139.954 110.109) (end 139.954 114.3) (width 0.1524) (layer B.Cu) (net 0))
 (segment (start 131.064 96.012) (end 131.318 96.266) (width 0.1524) (layer B.Cu) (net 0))
 (segment (start 131.318 101.473) (end 131.445 101.6) (width 0.1524) (layer B.Cu) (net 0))
 (segment (start 131.318 96.266) (end 131.318 101.473) (width 0.1524) (layer B.Cu) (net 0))
 (segment (start 131.445 101.6) (end 139.7 109.855) (width 0.1524) (layer B.Cu) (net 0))
 (segment (start 130.937 101.346) (end 130.937 101.6) (width 0.1524) (layer B.Cu) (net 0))
 (segment (start 130.937 101.346) (end 130.937 101.473) (width 0.1524) (layer B.Cu) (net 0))
 (segment (start 130.937 101.6) (end 139.573 110.236) (width 0.1524) (layer B.Cu) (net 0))
 (segment (start 139.573 114.427) (end 139.7 114.554) (width 0.1524) (layer B.Cu) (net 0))
 (segment (start 139.573 110.236) (end 139.573 114.427) (width 0.1524) (layer B.Cu) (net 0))
 (segment (start 147.955 91.694) (end 147.955 95.631) (width 0.1524) (layer B.Cu) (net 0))
 (segment (start 147.955 75.057) (end 147.955 91.694) (width 0.1524) (layer B.Cu) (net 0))
 (segment (start 148.336 91.694) (end 148.336 96.012) (width 0.1524) (layer B.Cu) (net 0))
 (segment (start 148.336 88.9) (end 148.336 91.694) (width 0.1524) (layer B.Cu) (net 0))
 (segment (start 147.955 91.694) (end 147.955 101.6) (width 0.1524) (layer B.Cu) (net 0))
 (segment (start 149.606 114.3) (end 149.86 114.554) (width 0.1524) (layer B.Cu) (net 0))
 (segment (start 149.606 103.251) (end 149.606 114.3) (width 0.1524) (layer B.Cu) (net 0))
 (segment (start 147.955 101.6) (end 149.606 103.251) (width 0.1524) (layer B.Cu) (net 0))
 (segment (start 149.987 114.427) (end 149.86 114.554) (width 0.1524) (layer B.Cu) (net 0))
 (segment (start 149.987 103.124) (end 149.987 114.427) (width 0.1524) (layer B.Cu) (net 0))
 (segment (start 148.336 91.694) (end 148.336 101.473) (width 0.1524) (layer B.Cu) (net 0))
 (segment (start 139.446 128.778) (end 139.7 129.032) (width 0.1524) (layer B.Cu) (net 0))
 (segment (start 139.446 123.952) (end 139.446 128.778) (width 0.1524) (layer B.Cu) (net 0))
 (segment (start 149.987 128.905) (end 149.86 129.032) (width 0.1524) (layer B.Cu) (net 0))
 (segment (start 140.97 78.74) (end 140.97 101.473) (width 0.1524) (layer B.Cu) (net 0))
 (segment (start 145.415 119.38) (end 149.987 123.952) (width 0.1524) (layer B.Cu) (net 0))
 (segment (start 148.59 71.12) (end 140.97 78.74) (width 0.1524) (layer B.Cu) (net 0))
 (segment (start 140.97 101.473) (end 145.415 105.918) (width 0.1524) (layer B.Cu) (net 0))
 (segment (start 149.987 123.952) (end 149.987 128.905) (width 0.1524) (layer B.Cu) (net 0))
 (segment (start 145.415 105.918) (end 145.415 119.38) (width 0.1524) (layer B.Cu) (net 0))
 (segment (start 149.606 128.778) (end 149.86 129.032) (width 0.1524) (layer B.Cu) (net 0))
 (segment (start 140.589 78.613) (end 140.589 101.6) (width 0.1524) (layer B.Cu) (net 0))
 (segment (start 140.589 101.6) (end 145.034 106.045) (width 0.1524) (layer B.Cu) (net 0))
 (segment (start 145.034 106.045) (end 145.034 119.507) (width 0.1524) (layer B.Cu) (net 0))
 (segment (start 148.082 71.12) (end 140.589 78.613) (width 0.1524) (layer B.Cu) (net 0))
 (segment (start 145.034 119.507) (end 149.606 124.079) (width 0.1524) (layer B.Cu) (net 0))
 (segment (start 149.606 124.079) (end 149.606 128.778) (width 0.1524) (layer B.Cu) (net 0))
 (segment (start 139.827 128.905) (end 139.7 129.032) (width 0.1524) (layer B.Cu) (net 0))
 (segment (start 140.208 102.235) (end 144.399 106.426) (width 0.1524) (layer B.Cu) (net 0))
 (segment (start 139.827 124.079) (end 139.827 128.905) (width 0.1524) (layer B.Cu) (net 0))
 (segment (start 144.399 119.507) (end 139.827 124.079) (width 0.1524) (layer B.Cu) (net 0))
 (segment (start 144.399 106.426) (end 144.399 119.507) (width 0.1524) (layer B.Cu) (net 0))
 (segment (start 130.937 96.012) (end 131.064 95.885) (width 0.1524) (layer B.Cu) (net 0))
 (segment (start 130.937 101.346) (end 130.937 96.012) (width 0.1524) (layer B.Cu) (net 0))
 (segment (start 148.336 101.473) (end 149.987 103.124) (width 0.1524) (layer B.Cu) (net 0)))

